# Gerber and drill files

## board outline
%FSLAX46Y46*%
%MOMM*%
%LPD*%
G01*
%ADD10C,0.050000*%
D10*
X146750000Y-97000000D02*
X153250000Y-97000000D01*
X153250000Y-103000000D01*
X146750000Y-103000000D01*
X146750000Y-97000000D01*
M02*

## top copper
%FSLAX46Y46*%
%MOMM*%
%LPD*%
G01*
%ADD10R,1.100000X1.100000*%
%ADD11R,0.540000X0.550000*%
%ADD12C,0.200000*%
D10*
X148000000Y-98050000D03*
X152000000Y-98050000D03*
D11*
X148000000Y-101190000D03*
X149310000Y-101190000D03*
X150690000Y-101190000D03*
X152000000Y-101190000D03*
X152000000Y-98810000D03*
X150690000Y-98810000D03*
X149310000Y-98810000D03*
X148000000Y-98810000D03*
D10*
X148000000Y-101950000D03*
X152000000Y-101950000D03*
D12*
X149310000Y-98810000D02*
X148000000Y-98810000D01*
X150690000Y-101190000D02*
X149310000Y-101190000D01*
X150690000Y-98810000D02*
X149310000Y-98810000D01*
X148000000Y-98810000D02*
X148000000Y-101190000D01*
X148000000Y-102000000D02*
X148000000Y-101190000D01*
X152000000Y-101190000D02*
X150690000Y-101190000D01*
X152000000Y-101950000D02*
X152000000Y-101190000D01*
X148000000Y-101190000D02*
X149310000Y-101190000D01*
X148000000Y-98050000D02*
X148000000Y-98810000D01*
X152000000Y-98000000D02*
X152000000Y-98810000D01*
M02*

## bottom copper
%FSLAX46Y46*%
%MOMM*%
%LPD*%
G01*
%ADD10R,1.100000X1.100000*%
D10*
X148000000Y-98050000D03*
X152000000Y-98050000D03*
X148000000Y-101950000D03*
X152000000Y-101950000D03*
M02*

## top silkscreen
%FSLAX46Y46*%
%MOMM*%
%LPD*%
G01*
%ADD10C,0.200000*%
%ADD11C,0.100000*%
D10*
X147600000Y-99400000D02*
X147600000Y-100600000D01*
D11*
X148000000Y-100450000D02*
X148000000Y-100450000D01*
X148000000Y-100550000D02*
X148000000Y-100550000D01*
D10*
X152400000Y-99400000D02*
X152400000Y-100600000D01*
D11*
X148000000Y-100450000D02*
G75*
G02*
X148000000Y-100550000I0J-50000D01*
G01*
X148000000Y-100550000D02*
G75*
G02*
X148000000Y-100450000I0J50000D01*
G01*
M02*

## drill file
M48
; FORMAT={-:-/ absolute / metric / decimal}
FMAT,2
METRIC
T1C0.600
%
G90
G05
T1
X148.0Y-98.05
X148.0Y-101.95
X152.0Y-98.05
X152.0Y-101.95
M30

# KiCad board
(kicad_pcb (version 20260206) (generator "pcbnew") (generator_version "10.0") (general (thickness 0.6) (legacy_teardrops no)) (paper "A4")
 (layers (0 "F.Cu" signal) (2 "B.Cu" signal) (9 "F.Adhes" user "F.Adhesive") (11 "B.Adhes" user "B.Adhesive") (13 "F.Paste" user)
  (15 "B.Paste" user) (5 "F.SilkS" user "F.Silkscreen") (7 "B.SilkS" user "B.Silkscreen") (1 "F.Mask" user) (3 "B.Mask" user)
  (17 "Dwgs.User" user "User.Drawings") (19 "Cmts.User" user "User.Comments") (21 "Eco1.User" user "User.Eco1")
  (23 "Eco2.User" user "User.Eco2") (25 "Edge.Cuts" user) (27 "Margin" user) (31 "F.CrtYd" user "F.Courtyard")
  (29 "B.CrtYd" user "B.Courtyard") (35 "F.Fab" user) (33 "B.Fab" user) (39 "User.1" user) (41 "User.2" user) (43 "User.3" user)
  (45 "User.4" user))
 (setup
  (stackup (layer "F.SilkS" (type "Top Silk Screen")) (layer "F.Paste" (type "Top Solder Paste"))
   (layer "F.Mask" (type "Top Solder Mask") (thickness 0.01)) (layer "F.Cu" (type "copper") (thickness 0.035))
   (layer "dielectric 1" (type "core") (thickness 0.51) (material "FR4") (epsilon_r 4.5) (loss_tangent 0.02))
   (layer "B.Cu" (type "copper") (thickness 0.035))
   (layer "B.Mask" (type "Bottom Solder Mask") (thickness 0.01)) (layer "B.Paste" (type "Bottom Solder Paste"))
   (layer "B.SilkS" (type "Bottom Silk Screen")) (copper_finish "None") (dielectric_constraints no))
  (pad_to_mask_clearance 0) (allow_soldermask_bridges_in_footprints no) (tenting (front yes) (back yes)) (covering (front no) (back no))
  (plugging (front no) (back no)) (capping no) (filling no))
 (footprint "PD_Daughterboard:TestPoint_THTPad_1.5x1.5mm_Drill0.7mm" (layer "F.Cu") (at 148 98.05)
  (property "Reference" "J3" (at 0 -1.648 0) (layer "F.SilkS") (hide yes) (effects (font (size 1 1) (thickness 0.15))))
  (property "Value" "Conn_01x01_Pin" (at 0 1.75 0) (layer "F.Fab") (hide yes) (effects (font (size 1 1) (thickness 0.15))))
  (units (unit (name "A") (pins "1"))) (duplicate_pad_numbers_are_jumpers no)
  (pad "1" thru_hole rect (at 0 0) (size 1.1 1.1) (drill 0.6) (layers "*.Cu" "*.Mask") (remove_unused_layers no) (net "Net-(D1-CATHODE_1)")))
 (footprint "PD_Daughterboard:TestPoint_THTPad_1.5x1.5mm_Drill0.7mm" (layer "F.Cu") (at 152 98.05)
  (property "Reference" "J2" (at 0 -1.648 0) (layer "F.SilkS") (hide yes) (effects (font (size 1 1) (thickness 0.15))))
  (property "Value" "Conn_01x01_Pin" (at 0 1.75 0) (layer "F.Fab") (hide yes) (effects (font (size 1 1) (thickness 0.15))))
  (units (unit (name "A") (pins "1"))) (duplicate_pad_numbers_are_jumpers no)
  (pad "1" thru_hole rect (at 0 0) (size 1.1 1.1) (drill 0.6) (layers "*.Cu" "*.Mask") (remove_unused_layers no) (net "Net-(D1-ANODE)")))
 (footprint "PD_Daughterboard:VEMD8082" (layer "F.Cu") (at 150 100)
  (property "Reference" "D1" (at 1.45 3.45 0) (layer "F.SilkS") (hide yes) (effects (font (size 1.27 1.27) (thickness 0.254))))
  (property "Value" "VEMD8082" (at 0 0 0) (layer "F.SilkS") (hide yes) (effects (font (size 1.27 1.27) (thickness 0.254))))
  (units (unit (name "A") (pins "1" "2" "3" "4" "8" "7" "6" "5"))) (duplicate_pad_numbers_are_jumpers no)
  (fp_line (start -2.4 -0.6) (end -2.4 0.6) (stroke (width 0.2) (type solid)) (layer "F.SilkS"))
  (fp_line (start -2 0.45) (end -2 0.45) (stroke (width 0.1) (type solid)) (layer "F.SilkS"))
  (fp_line (start -2 0.55) (end -2 0.55) (stroke (width 0.1) (type solid)) (layer "F.SilkS"))
  (fp_line (start 2.4 -0.6) (end 2.4 0.6) (stroke (width 0.2) (type solid)) (layer "F.SilkS"))
  (fp_arc (start -2 0.45) (mid -1.95 0.5) (end -2 0.55) (stroke (width 0.1) (type solid)) (layer "F.SilkS"))
  (fp_arc (start -2 0.55) (mid -2.05 0.5) (end -2 0.45) (stroke (width 0.1) (type solid)) (layer "F.SilkS"))
  (pad "1" smd rect (at -2 1.19) (size 0.54 0.55) (layers "F.Cu" "F.Mask" "F.Paste") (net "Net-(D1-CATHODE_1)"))
  (pad "2" smd rect (at -0.69 1.19) (size 0.54 0.55) (layers "F.Cu" "F.Mask" "F.Paste") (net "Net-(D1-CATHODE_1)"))
  (pad "3" smd rect (at 0.69 1.19) (size 0.54 0.55) (layers "F.Cu" "F.Mask" "F.Paste") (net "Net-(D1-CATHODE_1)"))
  (pad "4" smd rect (at 2 1.19) (size 0.54 0.55) (layers "F.Cu" "F.Mask" "F.Paste") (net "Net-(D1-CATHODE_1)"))
  (pad "5" smd rect (at 2 -1.19) (size 0.54 0.55) (layers "F.Cu" "F.Mask" "F.Paste") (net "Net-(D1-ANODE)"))
  (pad "6" smd rect (at 0.69 -1.19) (size 0.54 0.55) (layers "F.Cu" "F.Mask" "F.Paste") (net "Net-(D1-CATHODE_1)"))
  (pad "7" smd rect (at -0.69 -1.19) (size 0.54 0.55) (layers "F.Cu" "F.Mask" "F.Paste") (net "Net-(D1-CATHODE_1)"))
  (pad "8" smd rect (at -2 -1.19) (size 0.54 0.55) (layers "F.Cu" "F.Mask" "F.Paste") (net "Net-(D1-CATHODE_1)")))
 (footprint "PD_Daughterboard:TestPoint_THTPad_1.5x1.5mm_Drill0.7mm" (layer "F.Cu") (at 148 101.95)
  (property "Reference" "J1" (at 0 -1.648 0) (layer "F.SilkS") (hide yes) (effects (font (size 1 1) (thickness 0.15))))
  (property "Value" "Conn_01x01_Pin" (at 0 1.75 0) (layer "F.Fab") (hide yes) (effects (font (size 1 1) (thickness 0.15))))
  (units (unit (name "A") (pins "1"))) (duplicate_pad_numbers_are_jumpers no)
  (pad "1" thru_hole rect (at 0 0) (size 1.1 1.1) (drill 0.6) (layers "*.Cu" "*.Mask") (remove_unused_layers no) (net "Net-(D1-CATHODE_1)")))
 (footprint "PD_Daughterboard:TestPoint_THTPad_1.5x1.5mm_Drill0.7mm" (layer "F.Cu") (at 152 101.95)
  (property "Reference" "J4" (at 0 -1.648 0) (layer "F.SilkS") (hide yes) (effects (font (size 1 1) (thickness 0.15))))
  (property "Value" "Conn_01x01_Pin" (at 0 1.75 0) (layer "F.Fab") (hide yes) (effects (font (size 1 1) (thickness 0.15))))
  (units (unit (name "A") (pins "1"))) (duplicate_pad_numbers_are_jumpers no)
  (pad "1" thru_hole rect (at 0 0) (size 1.1 1.1) (drill 0.6) (layers "*.Cu" "*.Mask") (remove_unused_layers no) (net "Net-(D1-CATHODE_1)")))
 (gr_rect (start 146.75 97) (end 153.25 103) (stroke (width 0.05) (type default)) (fill no) (layer "Edge.Cuts"))
 (segment (start 149.31 98.81) (end 148 98.81) (width 0.2) (layer "F.Cu") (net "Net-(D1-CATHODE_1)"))
 (segment (start 150.69 101.19) (end 149.31 101.19) (width 0.2) (layer "F.Cu") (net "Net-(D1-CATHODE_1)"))
 (segment (start 150.69 98.81) (end 149.31 98.81) (width 0.2) (layer "F.Cu") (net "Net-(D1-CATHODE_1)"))
 (segment (start 148 98.81) (end 148 101.19) (width 0.2) (layer "F.Cu") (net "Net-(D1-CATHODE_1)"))
 (segment (start 148 102) (end 148 101.19) (width 0.2) (layer "F.Cu") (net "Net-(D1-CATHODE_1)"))
 (segment (start 152 101.19) (end 150.69 101.19) (width 0.2) (layer "F.Cu") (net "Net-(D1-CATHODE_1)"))
 (segment (start 152 101.95) (end 152 101.19) (width 0.2) (layer "F.Cu") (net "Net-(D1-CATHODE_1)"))
 (segment (start 148 101.19) (end 149.31 101.19) (width 0.2) (layer "F.Cu") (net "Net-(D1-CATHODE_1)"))
 (segment (start 148 98.05) (end 148 98.81) (width 0.2) (layer "F.Cu") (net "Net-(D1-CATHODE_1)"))
 (segment (start 152 98) (end 152 98.81) (width 0.2) (layer "F.Cu") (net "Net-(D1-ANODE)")))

